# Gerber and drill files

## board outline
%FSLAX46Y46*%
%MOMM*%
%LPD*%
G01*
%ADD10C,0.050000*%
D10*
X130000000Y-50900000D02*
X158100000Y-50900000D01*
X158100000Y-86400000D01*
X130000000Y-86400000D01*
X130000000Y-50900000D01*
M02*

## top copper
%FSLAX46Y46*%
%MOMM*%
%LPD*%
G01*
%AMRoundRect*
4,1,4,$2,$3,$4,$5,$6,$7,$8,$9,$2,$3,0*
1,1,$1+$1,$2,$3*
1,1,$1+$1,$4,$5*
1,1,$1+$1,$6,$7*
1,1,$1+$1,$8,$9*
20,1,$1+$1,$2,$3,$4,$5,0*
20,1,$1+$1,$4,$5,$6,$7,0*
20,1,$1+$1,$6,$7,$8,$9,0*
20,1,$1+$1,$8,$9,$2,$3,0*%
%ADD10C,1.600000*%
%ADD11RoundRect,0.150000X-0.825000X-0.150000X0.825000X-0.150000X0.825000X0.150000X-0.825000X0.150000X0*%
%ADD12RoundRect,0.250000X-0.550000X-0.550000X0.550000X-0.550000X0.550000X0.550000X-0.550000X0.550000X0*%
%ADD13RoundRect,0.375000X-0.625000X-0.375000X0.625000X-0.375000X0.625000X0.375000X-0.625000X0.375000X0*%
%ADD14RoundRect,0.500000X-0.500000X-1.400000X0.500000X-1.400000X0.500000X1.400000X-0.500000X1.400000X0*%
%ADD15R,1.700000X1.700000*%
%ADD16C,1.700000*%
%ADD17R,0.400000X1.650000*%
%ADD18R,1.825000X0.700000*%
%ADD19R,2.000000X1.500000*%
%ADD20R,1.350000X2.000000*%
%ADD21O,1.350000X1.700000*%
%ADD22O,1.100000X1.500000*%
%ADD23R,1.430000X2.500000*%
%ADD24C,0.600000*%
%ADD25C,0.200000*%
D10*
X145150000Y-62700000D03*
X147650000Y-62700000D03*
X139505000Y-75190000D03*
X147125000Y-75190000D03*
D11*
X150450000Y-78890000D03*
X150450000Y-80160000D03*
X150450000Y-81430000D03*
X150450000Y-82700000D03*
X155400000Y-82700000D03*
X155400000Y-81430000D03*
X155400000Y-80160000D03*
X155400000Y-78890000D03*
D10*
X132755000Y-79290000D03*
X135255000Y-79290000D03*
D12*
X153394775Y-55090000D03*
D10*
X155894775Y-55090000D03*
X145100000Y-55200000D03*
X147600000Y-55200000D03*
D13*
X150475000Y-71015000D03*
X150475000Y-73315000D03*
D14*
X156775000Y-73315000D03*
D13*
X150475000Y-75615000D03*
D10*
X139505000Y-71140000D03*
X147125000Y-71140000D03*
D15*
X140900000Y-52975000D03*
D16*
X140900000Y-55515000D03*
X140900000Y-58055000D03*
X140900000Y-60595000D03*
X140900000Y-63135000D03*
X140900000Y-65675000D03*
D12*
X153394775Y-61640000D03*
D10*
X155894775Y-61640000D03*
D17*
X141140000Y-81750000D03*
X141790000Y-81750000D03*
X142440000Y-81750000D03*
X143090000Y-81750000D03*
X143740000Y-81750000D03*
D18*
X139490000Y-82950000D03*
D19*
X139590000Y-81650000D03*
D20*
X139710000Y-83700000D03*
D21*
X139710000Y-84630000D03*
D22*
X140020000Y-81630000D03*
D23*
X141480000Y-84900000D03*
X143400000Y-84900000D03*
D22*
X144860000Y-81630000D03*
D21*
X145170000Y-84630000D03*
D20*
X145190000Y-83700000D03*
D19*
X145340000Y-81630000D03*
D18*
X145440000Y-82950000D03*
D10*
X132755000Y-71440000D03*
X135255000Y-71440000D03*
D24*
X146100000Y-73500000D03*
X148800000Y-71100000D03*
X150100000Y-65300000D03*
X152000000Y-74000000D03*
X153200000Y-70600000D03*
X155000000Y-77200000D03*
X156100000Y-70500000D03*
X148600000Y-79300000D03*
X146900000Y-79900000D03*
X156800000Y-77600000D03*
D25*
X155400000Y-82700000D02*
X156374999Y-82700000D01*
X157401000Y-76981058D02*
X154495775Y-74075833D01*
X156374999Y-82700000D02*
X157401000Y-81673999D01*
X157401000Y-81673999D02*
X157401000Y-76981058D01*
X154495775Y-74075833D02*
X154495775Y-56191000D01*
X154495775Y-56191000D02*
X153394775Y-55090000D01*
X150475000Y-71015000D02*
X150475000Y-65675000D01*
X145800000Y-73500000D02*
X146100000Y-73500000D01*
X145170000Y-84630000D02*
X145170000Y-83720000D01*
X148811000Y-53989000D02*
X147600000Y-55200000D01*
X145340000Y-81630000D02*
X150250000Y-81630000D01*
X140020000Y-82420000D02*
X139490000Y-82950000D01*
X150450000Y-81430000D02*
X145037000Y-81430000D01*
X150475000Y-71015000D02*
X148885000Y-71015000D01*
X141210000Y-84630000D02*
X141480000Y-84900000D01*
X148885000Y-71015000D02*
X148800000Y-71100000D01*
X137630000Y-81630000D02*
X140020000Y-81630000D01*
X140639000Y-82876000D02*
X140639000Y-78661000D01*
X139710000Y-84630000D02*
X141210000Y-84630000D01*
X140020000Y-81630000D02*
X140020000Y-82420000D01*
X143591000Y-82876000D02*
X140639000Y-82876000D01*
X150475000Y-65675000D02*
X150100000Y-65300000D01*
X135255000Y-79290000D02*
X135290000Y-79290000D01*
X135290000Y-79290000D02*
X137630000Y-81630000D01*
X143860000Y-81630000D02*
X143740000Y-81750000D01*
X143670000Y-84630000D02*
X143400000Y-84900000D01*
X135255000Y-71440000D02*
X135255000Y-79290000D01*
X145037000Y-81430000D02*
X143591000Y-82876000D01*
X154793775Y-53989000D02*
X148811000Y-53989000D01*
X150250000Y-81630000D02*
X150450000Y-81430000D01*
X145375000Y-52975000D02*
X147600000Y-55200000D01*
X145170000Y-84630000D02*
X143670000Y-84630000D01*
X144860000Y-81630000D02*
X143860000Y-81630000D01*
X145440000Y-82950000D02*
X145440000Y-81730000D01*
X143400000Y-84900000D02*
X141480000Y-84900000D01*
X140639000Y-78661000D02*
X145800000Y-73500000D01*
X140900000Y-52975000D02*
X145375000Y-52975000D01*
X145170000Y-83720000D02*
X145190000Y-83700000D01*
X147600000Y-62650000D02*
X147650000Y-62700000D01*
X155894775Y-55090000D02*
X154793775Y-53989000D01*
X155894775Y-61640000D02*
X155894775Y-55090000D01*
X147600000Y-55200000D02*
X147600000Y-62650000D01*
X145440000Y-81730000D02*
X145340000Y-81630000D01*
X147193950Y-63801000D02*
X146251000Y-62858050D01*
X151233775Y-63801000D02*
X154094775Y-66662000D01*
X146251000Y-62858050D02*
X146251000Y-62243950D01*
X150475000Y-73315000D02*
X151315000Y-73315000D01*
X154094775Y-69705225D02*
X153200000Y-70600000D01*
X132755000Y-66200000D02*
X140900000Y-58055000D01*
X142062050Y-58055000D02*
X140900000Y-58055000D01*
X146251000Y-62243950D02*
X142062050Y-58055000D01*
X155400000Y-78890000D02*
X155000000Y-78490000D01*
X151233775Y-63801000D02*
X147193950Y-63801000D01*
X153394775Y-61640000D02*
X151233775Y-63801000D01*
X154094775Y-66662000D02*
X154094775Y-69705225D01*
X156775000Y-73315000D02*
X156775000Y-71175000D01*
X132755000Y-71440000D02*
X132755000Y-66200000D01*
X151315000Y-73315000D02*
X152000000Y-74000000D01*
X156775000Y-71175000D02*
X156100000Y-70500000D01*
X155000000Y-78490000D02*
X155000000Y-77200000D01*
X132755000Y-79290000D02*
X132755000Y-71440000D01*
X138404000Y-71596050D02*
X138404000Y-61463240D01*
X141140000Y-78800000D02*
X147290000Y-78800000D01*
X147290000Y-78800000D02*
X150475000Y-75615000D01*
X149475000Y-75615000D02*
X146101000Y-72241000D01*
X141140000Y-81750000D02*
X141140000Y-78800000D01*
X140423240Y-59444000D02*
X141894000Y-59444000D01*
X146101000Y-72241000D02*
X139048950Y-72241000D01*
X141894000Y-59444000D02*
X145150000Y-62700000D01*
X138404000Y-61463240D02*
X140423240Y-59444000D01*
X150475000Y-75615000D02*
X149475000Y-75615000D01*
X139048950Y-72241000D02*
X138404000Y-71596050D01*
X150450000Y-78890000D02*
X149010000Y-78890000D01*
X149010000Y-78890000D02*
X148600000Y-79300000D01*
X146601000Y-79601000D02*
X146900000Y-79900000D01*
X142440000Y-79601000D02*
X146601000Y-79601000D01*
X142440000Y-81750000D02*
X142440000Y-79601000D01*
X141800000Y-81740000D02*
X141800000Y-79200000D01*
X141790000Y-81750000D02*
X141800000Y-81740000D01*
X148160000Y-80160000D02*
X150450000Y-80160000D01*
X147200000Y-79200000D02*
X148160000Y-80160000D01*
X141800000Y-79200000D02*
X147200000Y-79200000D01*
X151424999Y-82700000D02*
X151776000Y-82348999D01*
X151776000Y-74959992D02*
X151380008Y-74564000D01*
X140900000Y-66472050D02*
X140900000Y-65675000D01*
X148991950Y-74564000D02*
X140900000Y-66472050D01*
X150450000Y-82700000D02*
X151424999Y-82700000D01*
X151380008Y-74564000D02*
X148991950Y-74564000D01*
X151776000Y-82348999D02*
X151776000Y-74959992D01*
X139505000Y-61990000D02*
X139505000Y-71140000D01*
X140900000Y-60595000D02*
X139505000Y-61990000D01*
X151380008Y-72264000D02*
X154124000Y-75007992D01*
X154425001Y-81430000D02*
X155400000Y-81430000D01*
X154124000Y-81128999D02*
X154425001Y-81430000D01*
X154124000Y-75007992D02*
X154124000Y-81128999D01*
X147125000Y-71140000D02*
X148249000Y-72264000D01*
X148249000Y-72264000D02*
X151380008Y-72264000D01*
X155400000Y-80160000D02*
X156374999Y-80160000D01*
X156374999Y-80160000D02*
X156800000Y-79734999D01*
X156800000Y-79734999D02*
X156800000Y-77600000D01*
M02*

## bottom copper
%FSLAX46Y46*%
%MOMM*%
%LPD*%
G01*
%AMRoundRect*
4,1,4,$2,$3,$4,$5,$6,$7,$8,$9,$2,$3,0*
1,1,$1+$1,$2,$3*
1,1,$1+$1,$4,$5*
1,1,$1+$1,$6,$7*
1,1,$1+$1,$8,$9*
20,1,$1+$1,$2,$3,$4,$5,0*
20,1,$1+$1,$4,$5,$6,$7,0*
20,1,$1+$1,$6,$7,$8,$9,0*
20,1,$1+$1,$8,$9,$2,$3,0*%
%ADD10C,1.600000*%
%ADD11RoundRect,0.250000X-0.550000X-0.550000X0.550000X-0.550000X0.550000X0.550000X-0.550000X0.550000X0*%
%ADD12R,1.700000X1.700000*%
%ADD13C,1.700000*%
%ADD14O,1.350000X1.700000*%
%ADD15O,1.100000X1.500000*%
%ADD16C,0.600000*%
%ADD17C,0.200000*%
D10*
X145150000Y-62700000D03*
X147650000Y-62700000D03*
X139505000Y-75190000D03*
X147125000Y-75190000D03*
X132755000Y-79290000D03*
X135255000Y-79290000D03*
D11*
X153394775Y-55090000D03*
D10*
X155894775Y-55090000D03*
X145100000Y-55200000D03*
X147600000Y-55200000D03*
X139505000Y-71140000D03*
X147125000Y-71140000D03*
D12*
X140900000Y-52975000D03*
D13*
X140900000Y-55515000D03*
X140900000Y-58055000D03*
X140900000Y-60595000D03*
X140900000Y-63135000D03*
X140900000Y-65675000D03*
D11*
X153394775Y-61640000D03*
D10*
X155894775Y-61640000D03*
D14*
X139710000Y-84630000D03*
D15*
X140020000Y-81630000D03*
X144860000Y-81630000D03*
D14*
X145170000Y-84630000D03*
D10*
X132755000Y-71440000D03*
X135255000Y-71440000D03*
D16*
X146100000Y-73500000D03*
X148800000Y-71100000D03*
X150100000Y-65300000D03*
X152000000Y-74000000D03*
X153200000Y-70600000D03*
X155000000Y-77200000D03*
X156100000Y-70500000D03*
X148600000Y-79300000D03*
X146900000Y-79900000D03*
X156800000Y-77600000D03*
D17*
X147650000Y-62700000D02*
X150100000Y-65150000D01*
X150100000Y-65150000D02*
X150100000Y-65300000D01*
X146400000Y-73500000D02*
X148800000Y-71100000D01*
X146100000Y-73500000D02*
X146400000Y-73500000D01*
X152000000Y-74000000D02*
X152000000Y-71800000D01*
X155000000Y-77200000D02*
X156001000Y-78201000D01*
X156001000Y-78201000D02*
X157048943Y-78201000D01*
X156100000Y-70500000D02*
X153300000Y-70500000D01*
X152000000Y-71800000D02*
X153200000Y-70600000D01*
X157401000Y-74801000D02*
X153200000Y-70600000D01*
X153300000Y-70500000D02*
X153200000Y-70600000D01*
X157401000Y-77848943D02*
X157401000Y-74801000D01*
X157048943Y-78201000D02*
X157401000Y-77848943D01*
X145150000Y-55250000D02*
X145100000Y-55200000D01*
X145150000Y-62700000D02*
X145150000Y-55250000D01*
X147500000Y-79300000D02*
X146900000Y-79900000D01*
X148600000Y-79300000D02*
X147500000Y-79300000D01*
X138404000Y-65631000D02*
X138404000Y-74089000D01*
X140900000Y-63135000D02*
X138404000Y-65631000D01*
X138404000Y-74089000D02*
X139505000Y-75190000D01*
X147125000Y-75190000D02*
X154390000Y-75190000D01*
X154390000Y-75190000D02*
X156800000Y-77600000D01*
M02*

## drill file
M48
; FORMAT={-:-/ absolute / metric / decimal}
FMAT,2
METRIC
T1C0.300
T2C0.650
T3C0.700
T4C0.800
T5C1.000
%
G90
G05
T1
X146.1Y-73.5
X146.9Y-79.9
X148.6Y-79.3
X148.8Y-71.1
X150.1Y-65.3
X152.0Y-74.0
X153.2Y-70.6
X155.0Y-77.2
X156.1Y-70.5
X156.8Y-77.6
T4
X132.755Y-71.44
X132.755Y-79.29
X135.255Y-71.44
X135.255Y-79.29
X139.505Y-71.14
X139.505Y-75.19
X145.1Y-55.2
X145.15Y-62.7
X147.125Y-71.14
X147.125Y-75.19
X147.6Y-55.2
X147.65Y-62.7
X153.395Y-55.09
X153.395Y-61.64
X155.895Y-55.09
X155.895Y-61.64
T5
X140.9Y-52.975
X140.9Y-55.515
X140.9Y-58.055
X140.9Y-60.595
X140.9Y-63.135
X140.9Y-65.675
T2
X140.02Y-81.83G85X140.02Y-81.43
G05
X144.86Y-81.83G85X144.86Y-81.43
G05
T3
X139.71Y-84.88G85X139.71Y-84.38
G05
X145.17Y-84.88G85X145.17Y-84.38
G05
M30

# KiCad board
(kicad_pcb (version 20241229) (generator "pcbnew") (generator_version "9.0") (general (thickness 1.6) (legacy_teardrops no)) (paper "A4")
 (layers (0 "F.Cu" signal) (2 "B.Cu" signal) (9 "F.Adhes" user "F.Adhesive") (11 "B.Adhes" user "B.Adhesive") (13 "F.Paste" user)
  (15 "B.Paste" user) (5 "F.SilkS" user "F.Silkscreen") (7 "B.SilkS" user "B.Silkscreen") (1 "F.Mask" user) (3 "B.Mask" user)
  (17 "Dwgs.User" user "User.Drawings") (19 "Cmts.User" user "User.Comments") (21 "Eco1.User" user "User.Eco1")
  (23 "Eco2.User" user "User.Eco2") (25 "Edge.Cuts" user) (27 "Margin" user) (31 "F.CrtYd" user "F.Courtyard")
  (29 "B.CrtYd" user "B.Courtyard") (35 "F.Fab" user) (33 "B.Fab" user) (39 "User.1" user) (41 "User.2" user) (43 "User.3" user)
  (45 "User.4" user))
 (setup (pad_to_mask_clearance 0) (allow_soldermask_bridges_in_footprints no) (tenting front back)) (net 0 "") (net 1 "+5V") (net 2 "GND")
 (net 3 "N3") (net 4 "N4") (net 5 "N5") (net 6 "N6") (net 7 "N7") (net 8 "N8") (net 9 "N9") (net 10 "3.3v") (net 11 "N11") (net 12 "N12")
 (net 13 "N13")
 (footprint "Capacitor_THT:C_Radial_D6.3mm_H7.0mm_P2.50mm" (layer "F.Cu") (at 145.15 62.7)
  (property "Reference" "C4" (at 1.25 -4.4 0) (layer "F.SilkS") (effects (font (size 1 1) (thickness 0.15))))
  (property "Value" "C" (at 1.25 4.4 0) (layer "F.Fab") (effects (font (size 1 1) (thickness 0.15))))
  (pad "1" thru_hole circle (at 0 0) (size 1.6 1.6) (drill 0.8) (layers "*.Cu" "*.Mask") (remove_unused_layers no) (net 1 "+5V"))
  (pad "2" thru_hole circle (at 2.5 0) (size 1.6 1.6) (drill 0.8) (layers "*.Cu" "*.Mask") (remove_unused_layers no) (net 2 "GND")))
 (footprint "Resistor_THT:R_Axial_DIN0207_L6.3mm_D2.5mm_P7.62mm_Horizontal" (layer "F.Cu") (at 139.505 75.19)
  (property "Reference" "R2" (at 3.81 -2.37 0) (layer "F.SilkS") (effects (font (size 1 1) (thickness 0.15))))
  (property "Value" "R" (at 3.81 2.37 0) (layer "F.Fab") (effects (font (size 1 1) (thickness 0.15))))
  (pad "1" thru_hole circle (at 0 0) (size 1.6 1.6) (drill 0.8) (layers "*.Cu" "*.Mask") (remove_unused_layers no) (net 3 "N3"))
  (pad "2" thru_hole circle (at 7.62 0) (size 1.6 1.6) (drill 0.8) (layers "*.Cu" "*.Mask") (remove_unused_layers no) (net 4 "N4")))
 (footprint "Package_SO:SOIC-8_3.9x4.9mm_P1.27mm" (layer "F.Cu") (at 152.925 80.795)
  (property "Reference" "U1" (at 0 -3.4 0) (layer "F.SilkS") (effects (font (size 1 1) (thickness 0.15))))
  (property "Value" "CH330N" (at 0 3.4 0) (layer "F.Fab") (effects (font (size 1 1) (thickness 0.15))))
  (pad "1" smd roundrect (at -2.475 -1.905) (size 1.95 0.6) (layers "F.Cu" "F.Mask" "F.Paste") (roundrect_rratio 0.25) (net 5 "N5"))
  (pad "2" smd roundrect (at -2.475 -0.635) (size 1.95 0.6) (layers "F.Cu" "F.Mask" "F.Paste") (roundrect_rratio 0.25) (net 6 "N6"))
  (pad "3" smd roundrect (at -2.475 0.635) (size 1.95 0.6) (layers "F.Cu" "F.Mask" "F.Paste") (roundrect_rratio 0.25) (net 2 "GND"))
  (pad "4" smd roundrect (at -2.475 1.905) (size 1.95 0.6) (layers "F.Cu" "F.Mask" "F.Paste") (roundrect_rratio 0.25) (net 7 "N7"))
  (pad "5" smd roundrect (at 2.475 1.905) (size 1.95 0.6) (layers "F.Cu" "F.Mask" "F.Paste") (roundrect_rratio 0.25) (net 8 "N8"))
  (pad "6" smd roundrect (at 2.475 0.635) (size 1.95 0.6) (layers "F.Cu" "F.Mask" "F.Paste") (roundrect_rratio 0.25) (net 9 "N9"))
  (pad "7" smd roundrect (at 2.475 -0.635) (size 1.95 0.6) (layers "F.Cu" "F.Mask" "F.Paste") (roundrect_rratio 0.25) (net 4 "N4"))
  (pad "8" smd roundrect (at 2.475 -1.905) (size 1.95 0.6) (layers "F.Cu" "F.Mask" "F.Paste") (roundrect_rratio 0.25) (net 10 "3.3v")))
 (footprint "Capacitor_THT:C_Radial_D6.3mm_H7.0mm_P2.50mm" (layer "F.Cu") (at 132.755 79.29)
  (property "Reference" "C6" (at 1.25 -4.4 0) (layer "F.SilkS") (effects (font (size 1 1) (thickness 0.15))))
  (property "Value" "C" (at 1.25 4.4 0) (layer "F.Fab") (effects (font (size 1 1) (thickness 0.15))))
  (pad "1" thru_hole circle (at 0 0) (size 1.6 1.6) (drill 0.8) (layers "*.Cu" "*.Mask") (remove_unused_layers no) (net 10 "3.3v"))
  (pad "2" thru_hole circle (at 2.5 0) (size 1.6 1.6) (drill 0.8) (layers "*.Cu" "*.Mask") (remove_unused_layers no) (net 2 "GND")))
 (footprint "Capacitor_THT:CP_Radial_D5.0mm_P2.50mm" (layer "F.Cu") (at 153.394775 55.09)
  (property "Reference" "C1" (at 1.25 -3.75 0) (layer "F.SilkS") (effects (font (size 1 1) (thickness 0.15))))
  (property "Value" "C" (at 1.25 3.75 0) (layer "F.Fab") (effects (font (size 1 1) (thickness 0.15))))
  (pad "1" thru_hole roundrect (at 0 0) (size 1.6 1.6) (drill 0.8) (layers "*.Cu" "*.Mask") (remove_unused_layers no)
   (roundrect_rratio 0.15625) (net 8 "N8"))
  (pad "2" thru_hole circle (at 2.5 0) (size 1.6 1.6) (drill 0.8) (layers "*.Cu" "*.Mask") (remove_unused_layers no) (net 2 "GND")))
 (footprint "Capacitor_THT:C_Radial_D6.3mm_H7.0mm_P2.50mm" (layer "F.Cu") (at 145.1 55.2)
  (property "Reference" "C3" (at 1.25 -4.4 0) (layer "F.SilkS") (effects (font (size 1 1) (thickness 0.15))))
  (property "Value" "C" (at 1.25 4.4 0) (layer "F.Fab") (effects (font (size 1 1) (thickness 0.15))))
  (pad "1" thru_hole circle (at 0 0) (size 1.6 1.6) (drill 0.8) (layers "*.Cu" "*.Mask") (remove_unused_layers no) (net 1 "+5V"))
  (pad "2" thru_hole circle (at 2.5 0) (size 1.6 1.6) (drill 0.8) (layers "*.Cu" "*.Mask") (remove_unused_layers no) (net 2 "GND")))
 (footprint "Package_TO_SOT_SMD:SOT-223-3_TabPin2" (layer "F.Cu") (at 153.625 73.315)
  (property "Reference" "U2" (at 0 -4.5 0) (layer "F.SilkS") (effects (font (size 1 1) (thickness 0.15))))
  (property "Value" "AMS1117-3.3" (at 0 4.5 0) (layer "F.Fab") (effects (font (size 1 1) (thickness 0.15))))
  (pad "1" smd roundrect (at -3.15 -2.3) (size 2 1.5) (layers "F.Cu" "F.Mask" "F.Paste") (roundrect_rratio 0.25) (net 2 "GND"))
  (pad "2" smd roundrect (at -3.15 0) (size 2 1.5) (layers "F.Cu" "F.Mask" "F.Paste") (roundrect_rratio 0.25) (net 10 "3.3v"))
  (pad "2" smd roundrect (at 3.15 0) (size 2 3.8) (layers "F.Cu" "F.Mask" "F.Paste") (roundrect_rratio 0.25) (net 10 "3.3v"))
  (pad "3" smd roundrect (at -3.15 2.3) (size 2 1.5) (layers "F.Cu" "F.Mask" "F.Paste") (roundrect_rratio 0.25) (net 1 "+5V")))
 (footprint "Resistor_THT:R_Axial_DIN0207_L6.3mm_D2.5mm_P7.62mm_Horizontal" (layer "F.Cu") (at 139.505 71.14)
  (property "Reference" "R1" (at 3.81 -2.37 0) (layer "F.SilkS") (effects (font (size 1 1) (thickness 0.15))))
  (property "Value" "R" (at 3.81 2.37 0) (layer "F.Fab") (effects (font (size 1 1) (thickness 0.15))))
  (pad "1" thru_hole circle (at 0 0) (size 1.6 1.6) (drill 0.8) (layers "*.Cu" "*.Mask") (remove_unused_layers no) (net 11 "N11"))
  (pad "2" thru_hole circle (at 7.62 0) (size 1.6 1.6) (drill 0.8) (layers "*.Cu" "*.Mask") (remove_unused_layers no) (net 9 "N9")))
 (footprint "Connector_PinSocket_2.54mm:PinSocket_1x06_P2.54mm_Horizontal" (layer "F.Cu") (at 140.9 52.975)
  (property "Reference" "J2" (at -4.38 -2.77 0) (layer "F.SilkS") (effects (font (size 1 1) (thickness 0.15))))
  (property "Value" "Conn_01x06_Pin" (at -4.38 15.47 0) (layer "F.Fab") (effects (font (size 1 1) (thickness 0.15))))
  (pad "1" thru_hole rect (at 0 0) (size 1.7 1.7) (drill 1) (layers "*.Cu" "*.Mask") (remove_unused_layers no) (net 2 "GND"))
  (pad "2" thru_hole circle (at 0 2.54) (size 1.7 1.7) (drill 1) (layers "*.Cu" "*.Mask") (remove_unused_layers no) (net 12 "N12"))
  (pad "3" thru_hole circle (at 0 5.08) (size 1.7 1.7) (drill 1) (layers "*.Cu" "*.Mask") (remove_unused_layers no) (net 10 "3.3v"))
  (pad "4" thru_hole circle (at 0 7.62) (size 1.7 1.7) (drill 1) (layers "*.Cu" "*.Mask") (remove_unused_layers no) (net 11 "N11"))
  (pad "5" thru_hole circle (at 0 10.16) (size 1.7 1.7) (drill 1) (layers "*.Cu" "*.Mask") (remove_unused_layers no) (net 3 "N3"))
  (pad "6" thru_hole circle (at 0 12.7) (size 1.7 1.7) (drill 1) (layers "*.Cu" "*.Mask") (remove_unused_layers no) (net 7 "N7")))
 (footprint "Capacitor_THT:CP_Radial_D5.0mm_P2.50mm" (layer "F.Cu") (at 153.394775 61.64)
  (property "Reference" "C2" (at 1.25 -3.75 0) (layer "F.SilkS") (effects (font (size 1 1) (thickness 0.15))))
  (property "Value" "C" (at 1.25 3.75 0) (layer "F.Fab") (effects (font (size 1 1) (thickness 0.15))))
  (pad "1" thru_hole roundrect (at 0 0) (size 1.6 1.6) (drill 0.8) (layers "*.Cu" "*.Mask") (remove_unused_layers no)
   (roundrect_rratio 0.15625) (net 10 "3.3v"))
  (pad "2" thru_hole circle (at 2.5 0) (size 1.6 1.6) (drill 0.8) (layers "*.Cu" "*.Mask") (remove_unused_layers no) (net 2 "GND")))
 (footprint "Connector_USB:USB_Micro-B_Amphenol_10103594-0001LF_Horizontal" (layer "F.Cu") (at 142.465 83.515)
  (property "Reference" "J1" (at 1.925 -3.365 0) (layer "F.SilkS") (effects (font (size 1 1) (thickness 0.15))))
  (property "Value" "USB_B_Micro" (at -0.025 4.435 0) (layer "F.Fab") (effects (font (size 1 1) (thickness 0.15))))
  (pad "1" smd rect (at -1.325 -1.765 90) (size 1.65 0.4) (layers "F.Cu" "F.Mask" "F.Paste") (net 1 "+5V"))
  (pad "2" smd rect (at -0.675 -1.765 90) (size 1.65 0.4) (layers "F.Cu" "F.Mask" "F.Paste") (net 6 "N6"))
  (pad "3" smd rect (at -0.025 -1.765 90) (size 1.65 0.4) (layers "F.Cu" "F.Mask" "F.Paste") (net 5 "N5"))
  (pad "4" smd rect (at 0.625 -1.765 90) (size 1.65 0.4) (layers "F.Cu" "F.Mask" "F.Paste") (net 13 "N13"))
  (pad "5" smd rect (at 1.275 -1.765 90) (size 1.65 0.4) (layers "F.Cu" "F.Mask" "F.Paste") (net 2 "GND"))
  (pad "6" smd rect (at -2.975 -0.565) (size 1.825 0.7) (layers "F.Cu" "F.Mask" "F.Paste") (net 2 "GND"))
  (pad "6" smd rect (at -2.875 -1.865) (size 2 1.5) (layers "F.Cu" "F.Mask" "F.Paste") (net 2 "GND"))
  (pad "6" smd rect (at -2.755 0.185) (size 1.35 2) (layers "F.Cu" "F.Mask" "F.Paste") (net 2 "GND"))
  (pad "6" thru_hole oval (at -2.755 1.115 90) (size 1.7 1.35) (drill oval 1.2 0.7) (layers "*.Cu" "*.Mask") (remove_unused_layers no)
   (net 2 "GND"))
  (pad "6" thru_hole oval (at -2.445 -1.885 90) (size 1.5 1.1) (drill oval 1.05 0.65) (layers "*.Cu" "*.Mask") (remove_unused_layers no)
   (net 2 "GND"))
  (pad "6" smd rect (at -0.985 1.385 90) (size 2.5 1.43) (layers "F.Cu" "F.Mask" "F.Paste") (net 2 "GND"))
  (pad "6" smd rect (at 0.935 1.385 90) (size 2.5 1.43) (layers "F.Cu" "F.Mask" "F.Paste") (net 2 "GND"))
  (pad "6" thru_hole oval (at 2.395 -1.885 90) (size 1.5 1.1) (drill oval 1.05 0.65) (layers "*.Cu" "*.Mask") (remove_unused_layers no)
   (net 2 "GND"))
  (pad "6" thru_hole oval (at 2.705 1.115 90) (size 1.7 1.35) (drill oval 1.2 0.7) (layers "*.Cu" "*.Mask") (remove_unused_layers no)
   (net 2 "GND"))
  (pad "6" smd rect (at 2.725 0.185) (size 1.35 2) (layers "F.Cu" "F.Mask" "F.Paste") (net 2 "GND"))
  (pad "6" smd rect (at 2.875 -1.885) (size 2 1.5) (layers "F.Cu" "F.Mask" "F.Paste") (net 2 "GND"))
  (pad "6" smd rect (at 2.975 -0.565) (size 1.825 0.7) (layers "F.Cu" "F.Mask" "F.Paste") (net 2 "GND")))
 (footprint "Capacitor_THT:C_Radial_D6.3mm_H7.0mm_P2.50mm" (layer "F.Cu") (at 132.755 71.44)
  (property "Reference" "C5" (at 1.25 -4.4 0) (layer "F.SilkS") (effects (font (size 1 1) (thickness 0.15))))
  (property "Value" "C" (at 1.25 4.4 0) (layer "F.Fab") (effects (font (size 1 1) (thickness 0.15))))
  (pad "1" thru_hole circle (at 0 0) (size 1.6 1.6) (drill 0.8) (layers "*.Cu" "*.Mask") (remove_unused_layers no) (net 10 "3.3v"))
  (pad "2" thru_hole circle (at 2.5 0) (size 1.6 1.6) (drill 0.8) (layers "*.Cu" "*.Mask") (remove_unused_layers no) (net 2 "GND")))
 (gr_rect (start 130 50.9) (end 158.1 86.4) (stroke (width 0.05) (type default)) (fill no) (layer "Edge.Cuts"))
 (segment (start 155.4 82.7) (end 156.374999 82.7) (width 0.2) (layer "F.Cu") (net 8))
 (segment (start 157.401 76.981058) (end 154.495775 74.075833) (width 0.2) (layer "F.Cu") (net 8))
 (segment (start 156.374999 82.7) (end 157.401 81.673999) (width 0.2) (layer "F.Cu") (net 8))
 (segment (start 157.401 81.673999) (end 157.401 76.981058) (width 0.2) (layer "F.Cu") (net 8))
 (segment (start 154.495775 74.075833) (end 154.495775 56.191) (width 0.2) (layer "F.Cu") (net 8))
 (segment (start 154.495775 56.191) (end 153.394775 55.09) (width 0.2) (layer "F.Cu") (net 8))
 (segment (start 150.475 71.015) (end 150.475 65.675) (width 0.2) (layer "F.Cu") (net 2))
 (segment (start 145.8 73.5) (end 146.1 73.5) (width 0.2) (layer "F.Cu") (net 2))
 (segment (start 145.17 84.63) (end 145.17 83.72) (width 0.2) (layer "F.Cu") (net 2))
 (segment (start 148.811 53.989) (end 147.6 55.2) (width 0.2) (layer "F.Cu") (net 2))
 (segment (start 145.34 81.63) (end 150.25 81.63) (width 0.2) (layer "F.Cu") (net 2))
 (segment (start 140.02 82.42) (end 139.49 82.95) (width 0.2) (layer "F.Cu") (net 2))
 (segment (start 150.45 81.43) (end 145.037 81.43) (width 0.2) (layer "F.Cu") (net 2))
 (segment (start 150.475 71.015) (end 148.885 71.015) (width 0.2) (layer "F.Cu") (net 2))
 (segment (start 141.21 84.63) (end 141.48 84.9) (width 0.2) (layer "F.Cu") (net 2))
 (segment (start 148.885 71.015) (end 148.8 71.1) (width 0.2) (layer "F.Cu") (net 2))
 (segment (start 137.63 81.63) (end 140.02 81.63) (width 0.2) (layer "F.Cu") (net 2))
 (segment (start 140.639 82.876) (end 140.639 78.661) (width 0.2) (layer "F.Cu") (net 2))
 (segment (start 139.71 84.63) (end 141.21 84.63) (width 0.2) (layer "F.Cu") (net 2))
 (segment (start 140.02 81.63) (end 140.02 82.42) (width 0.2) (layer "F.Cu") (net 2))
 (segment (start 143.591 82.876) (end 140.639 82.876) (width 0.2) (layer "F.Cu") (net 2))
 (segment (start 150.475 65.675) (end 150.1 65.3) (width 0.2) (layer "F.Cu") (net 2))
 (segment (start 135.255 79.29) (end 135.29 79.29) (width 0.2) (layer "F.Cu") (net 2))
 (segment (start 135.29 79.29) (end 137.63 81.63) (width 0.2) (layer "F.Cu") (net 2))
 (segment (start 143.86 81.63) (end 143.74 81.75) (width 0.2) (layer "F.Cu") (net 2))
 (segment (start 143.67 84.63) (end 143.4 84.9) (width 0.2) (layer "F.Cu") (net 2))
 (segment (start 135.255 71.44) (end 135.255 79.29) (width 0.2) (layer "F.Cu") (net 2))
 (segment (start 145.037 81.43) (end 143.591 82.876) (width 0.2) (layer "F.Cu") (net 2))
 (segment (start 154.793775 53.989) (end 148.811 53.989) (width 0.2) (layer "F.Cu") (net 2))
 (segment (start 150.25 81.63) (end 150.45 81.43) (width 0.2) (layer "F.Cu") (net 2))
 (segment (start 145.375 52.975) (end 147.6 55.2) (width 0.2) (layer "F.Cu") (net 2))
 (segment (start 145.17 84.63) (end 143.67 84.63) (width 0.2) (layer "F.Cu") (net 2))
 (segment (start 144.86 81.63) (end 143.86 81.63) (width 0.2) (layer "F.Cu") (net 2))
 (segment (start 145.44 82.95) (end 145.44 81.73) (width 0.2) (layer "F.Cu") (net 2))
 (segment (start 143.4 84.9) (end 141.48 84.9) (width 0.2) (layer "F.Cu") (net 2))
 (segment (start 140.639 78.661) (end 145.8 73.5) (width 0.2) (layer "F.Cu") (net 2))
 (segment (start 140.9 52.975) (end 145.375 52.975) (width 0.2) (layer "F.Cu") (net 2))
 (segment (start 145.17 83.72) (end 145.19 83.7) (width 0.2) (layer "F.Cu") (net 2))
 (segment (start 147.6 62.65) (end 147.65 62.7) (width 0.2) (layer "F.Cu") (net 2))
 (segment (start 155.894775 55.09) (end 154.793775 53.989) (width 0.2) (layer "F.Cu") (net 2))
 (segment (start 155.894775 61.64) (end 155.894775 55.09) (width 0.2) (layer "F.Cu") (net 2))
 (segment (start 147.6 55.2) (end 147.6 62.65) (width 0.2) (layer "F.Cu") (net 2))
 (segment (start 145.44 81.73) (end 145.34 81.63) (width 0.2) (layer "F.Cu") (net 2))
 (via (at 146.1 73.5) (size 0.6) (drill 0.3) (layers "F.Cu" "B.Cu") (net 2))
 (via (at 148.8 71.1) (size 0.6) (drill 0.3) (layers "F.Cu" "B.Cu") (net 2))
 (via (at 150.1 65.3) (size 0.6) (drill 0.3) (layers "F.Cu" "B.Cu") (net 2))
 (segment (start 147.65 62.7) (end 150.1 65.15) (width 0.2) (layer "B.Cu") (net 2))
 (segment (start 150.1 65.15) (end 150.1 65.3) (width 0.2) (layer "B.Cu") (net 2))
 (segment (start 146.4 73.5) (end 148.8 71.1) (width 0.2) (layer "B.Cu") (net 2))
 (segment (start 146.1 73.5) (end 146.4 73.5) (width 0.2) (layer "B.Cu") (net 2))
 (segment (start 147.19395 63.801) (end 146.251 62.85805) (width 0.2) (layer "F.Cu") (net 10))
 (segment (start 151.233775 63.801) (end 154.094775 66.662) (width 0.2) (layer "F.Cu") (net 10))
 (segment (start 146.251 62.85805) (end 146.251 62.24395) (width 0.2) (layer "F.Cu") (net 10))
 (segment (start 150.475 73.315) (end 151.315 73.315) (width 0.2) (layer "F.Cu") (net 10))
 (segment (start 154.094775 69.705225) (end 153.2 70.6) (width 0.2) (layer "F.Cu") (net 10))
 (segment (start 132.755 66.2) (end 140.9 58.055) (width 0.2) (layer "F.Cu") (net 10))
 (segment (start 142.06205 58.055) (end 140.9 58.055) (width 0.2) (layer "F.Cu") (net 10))
 (segment (start 146.251 62.24395) (end 142.06205 58.055) (width 0.2) (layer "F.Cu") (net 10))
 (segment (start 155.4 78.89) (end 155 78.49) (width 0.2) (layer "F.Cu") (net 10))
 (segment (start 151.233775 63.801) (end 147.19395 63.801) (width 0.2) (layer "F.Cu") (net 10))
 (segment (start 153.394775 61.64) (end 151.233775 63.801) (width 0.2) (layer "F.Cu") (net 10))
 (segment (start 154.094775 66.662) (end 154.094775 69.705225) (width 0.2) (layer "F.Cu") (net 10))
 (segment (start 156.775 73.315) (end 156.775 71.175) (width 0.2) (layer "F.Cu") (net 10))
 (segment (start 132.755 71.44) (end 132.755 66.2) (width 0.2) (layer "F.Cu") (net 10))
 (segment (start 151.315 73.315) (end 152 74) (width 0.2) (layer "F.Cu") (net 10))
 (segment (start 156.775 71.175) (end 156.1 70.5) (width 0.2) (layer "F.Cu") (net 10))
 (segment (start 155 78.49) (end 155 77.2) (width 0.2) (layer "F.Cu") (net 10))
 (segment (start 132.755 79.29) (end 132.755 71.44) (width 0.2) (layer "F.Cu") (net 10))
 (via (at 152 74) (size 0.6) (drill 0.3) (layers "F.Cu" "B.Cu") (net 10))
 (via (at 153.2 70.6) (size 0.6) (drill 0.3) (layers "F.Cu" "B.Cu") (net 10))
 (via (at 155 77.2) (size 0.6) (drill 0.3) (layers "F.Cu" "B.Cu") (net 10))
 (via (at 156.1 70.5) (size 0.6) (drill 0.3) (layers "F.Cu" "B.Cu") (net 10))
 (segment (start 152 74) (end 152 71.8) (width 0.2) (layer "B.Cu") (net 10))
 (segment (start 155 77.2) (end 156.001 78.201) (width 0.2) (layer "B.Cu") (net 10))
 (segment (start 156.001 78.201) (end 157.048943 78.201) (width 0.2) (layer "B.Cu") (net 10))
 (segment (start 156.1 70.5) (end 153.3 70.5) (width 0.2) (layer "B.Cu") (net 10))
 (segment (start 152 71.8) (end 153.2 70.6) (width 0.2) (layer "B.Cu") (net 10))
 (segment (start 157.401 74.801) (end 153.2 70.6) (width 0.2) (layer "B.Cu") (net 10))
 (segment (start 153.3 70.5) (end 153.2 70.6) (width 0.2) (layer "B.Cu") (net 10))
 (segment (start 157.401 77.848943) (end 157.401 74.801) (width 0.2) (layer "B.Cu") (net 10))
 (segment (start 157.048943 78.201) (end 157.401 77.848943) (width 0.2) (layer "B.Cu") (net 10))
 (segment (start 138.404 71.59605) (end 138.404 61.46324) (width 0.2) (layer "F.Cu") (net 1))
 (segment (start 141.14 78.8) (end 147.29 78.8) (width 0.2) (layer "F.Cu") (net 1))
 (segment (start 147.29 78.8) (end 150.475 75.615) (width 0.2) (layer "F.Cu") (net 1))
 (segment (start 149.475 75.615) (end 146.101 72.241) (width 0.2) (layer "F.Cu") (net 1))
 (segment (start 141.14 81.75) (end 141.14 78.8) (width 0.2) (layer "F.Cu") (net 1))
 (segment (start 140.42324 59.444) (end 141.894 59.444) (width 0.2) (layer "F.Cu") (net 1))
 (segment (start 146.101 72.241) (end 139.04895 72.241) (width 0.2) (layer "F.Cu") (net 1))
 (segment (start 141.894 59.444) (end 145.15 62.7) (width 0.2) (layer "F.Cu") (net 1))
 (segment (start 138.404 61.46324) (end 140.42324 59.444) (width 0.2) (layer "F.Cu") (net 1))
 (segment (start 150.475 75.615) (end 149.475 75.615) (width 0.2) (layer "F.Cu") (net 1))
 (segment (start 139.04895 72.241) (end 138.404 71.59605) (width 0.2) (layer "F.Cu") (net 1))
 (segment (start 145.15 55.25) (end 145.1 55.2) (width 0.2) (layer "B.Cu") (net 1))
 (segment (start 145.15 62.7) (end 145.15 55.25) (width 0.2) (layer "B.Cu") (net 1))
 (segment (start 150.45 78.89) (end 149.01 78.89) (width 0.2) (layer "F.Cu") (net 5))
 (segment (start 149.01 78.89) (end 148.6 79.3) (width 0.2) (layer "F.Cu") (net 5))
 (segment (start 146.601 79.601) (end 146.9 79.9) (width 0.2) (layer "F.Cu") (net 5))
 (segment (start 142.44 79.601) (end 146.601 79.601) (width 0.2) (layer "F.Cu") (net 5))
 (segment (start 142.44 81.75) (end 142.44 79.601) (width 0.2) (layer "F.Cu") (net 5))
 (via (at 148.6 79.3) (size 0.6) (drill 0.3) (layers "F.Cu" "B.Cu") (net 5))
 (via (at 146.9 79.9) (size 0.6) (drill 0.3) (layers "F.Cu" "B.Cu") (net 5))
 (segment (start 147.5 79.3) (end 146.9 79.9) (width 0.2) (layer "B.Cu") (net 5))
 (segment (start 148.6 79.3) (end 147.5 79.3) (width 0.2) (layer "B.Cu") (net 5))
 (segment (start 141.8 81.74) (end 141.8 79.2) (width 0.2) (layer "F.Cu") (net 6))
 (segment (start 141.79 81.75) (end 141.8 81.74) (width 0.2) (layer "F.Cu") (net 6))
 (segment (start 148.16 80.16) (end 150.45 80.16) (width 0.2) (layer "F.Cu") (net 6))
 (segment (start 147.2 79.2) (end 148.16 80.16) (width 0.2) (layer "F.Cu") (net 6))
 (segment (start 141.8 79.2) (end 147.2 79.2) (width 0.2) (layer "F.Cu") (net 6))
 (segment (start 138.404 65.631) (end 138.404 74.089) (width 0.2) (layer "B.Cu") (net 3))
 (segment (start 140.9 63.135) (end 138.404 65.631) (width 0.2) (layer "B.Cu") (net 3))
 (segment (start 138.404 74.089) (end 139.505 75.19) (width 0.2) (layer "B.Cu") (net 3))
 (segment (start 151.424999 82.7) (end 151.776 82.348999) (width 0.2) (layer "F.Cu") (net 7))
 (segment (start 151.776 74.959992) (end 151.380008 74.564) (width 0.2) (layer "F.Cu") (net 7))
 (segment (start 140.9 66.47205) (end 140.9 65.675) (width 0.2) (layer "F.Cu") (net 7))
 (segment (start 148.99195 74.564) (end 140.9 66.47205) (width 0.2) (layer "F.Cu") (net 7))
 (segment (start 150.45 82.7) (end 151.424999 82.7) (width 0.2) (layer "F.Cu") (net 7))
 (segment (start 151.380008 74.564) (end 148.99195 74.564) (width 0.2) (layer "F.Cu") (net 7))
 (segment (start 151.776 82.348999) (end 151.776 74.959992) (width 0.2) (layer "F.Cu") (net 7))
 (segment (start 139.505 61.99) (end 139.505 71.14) (width 0.2) (layer "F.Cu") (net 11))
 (segment (start 140.9 60.595) (end 139.505 61.99) (width 0.2) (layer "F.Cu") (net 11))
 (segment (start 151.380008 72.264) (end 154.124 75.007992) (width 0.2) (layer "F.Cu") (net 9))
 (segment (start 154.425001 81.43) (end 155.4 81.43) (width 0.2) (layer "F.Cu") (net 9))
 (segment (start 154.124 81.128999) (end 154.425001 81.43) (width 0.2) (layer "F.Cu") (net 9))
 (segment (start 154.124 75.007992) (end 154.124 81.128999) (width 0.2) (layer "F.Cu") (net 9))
 (segment (start 147.125 71.14) (end 148.249 72.264) (width 0.2) (layer "F.Cu") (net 9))
 (segment (start 148.249 72.264) (end 151.380008 72.264) (width 0.2) (layer "F.Cu") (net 9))
 (segment (start 155.4 80.16) (end 156.374999 80.16) (width 0.2) (layer "F.Cu") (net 4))
 (segment (start 156.374999 80.16) (end 156.8 79.734999) (width 0.2) (layer "F.Cu") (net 4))
 (segment (start 156.8 79.734999) (end 156.8 77.6) (width 0.2) (layer "F.Cu") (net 4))
 (via (at 156.8 77.6) (size 0.6) (drill 0.3) (layers "F.Cu" "B.Cu") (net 4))
 (segment (start 147.125 75.19) (end 154.39 75.19) (width 0.2) (layer "B.Cu") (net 4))
 (segment (start 154.39 75.19) (end 156.8 77.6) (width 0.2) (layer "B.Cu") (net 4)))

